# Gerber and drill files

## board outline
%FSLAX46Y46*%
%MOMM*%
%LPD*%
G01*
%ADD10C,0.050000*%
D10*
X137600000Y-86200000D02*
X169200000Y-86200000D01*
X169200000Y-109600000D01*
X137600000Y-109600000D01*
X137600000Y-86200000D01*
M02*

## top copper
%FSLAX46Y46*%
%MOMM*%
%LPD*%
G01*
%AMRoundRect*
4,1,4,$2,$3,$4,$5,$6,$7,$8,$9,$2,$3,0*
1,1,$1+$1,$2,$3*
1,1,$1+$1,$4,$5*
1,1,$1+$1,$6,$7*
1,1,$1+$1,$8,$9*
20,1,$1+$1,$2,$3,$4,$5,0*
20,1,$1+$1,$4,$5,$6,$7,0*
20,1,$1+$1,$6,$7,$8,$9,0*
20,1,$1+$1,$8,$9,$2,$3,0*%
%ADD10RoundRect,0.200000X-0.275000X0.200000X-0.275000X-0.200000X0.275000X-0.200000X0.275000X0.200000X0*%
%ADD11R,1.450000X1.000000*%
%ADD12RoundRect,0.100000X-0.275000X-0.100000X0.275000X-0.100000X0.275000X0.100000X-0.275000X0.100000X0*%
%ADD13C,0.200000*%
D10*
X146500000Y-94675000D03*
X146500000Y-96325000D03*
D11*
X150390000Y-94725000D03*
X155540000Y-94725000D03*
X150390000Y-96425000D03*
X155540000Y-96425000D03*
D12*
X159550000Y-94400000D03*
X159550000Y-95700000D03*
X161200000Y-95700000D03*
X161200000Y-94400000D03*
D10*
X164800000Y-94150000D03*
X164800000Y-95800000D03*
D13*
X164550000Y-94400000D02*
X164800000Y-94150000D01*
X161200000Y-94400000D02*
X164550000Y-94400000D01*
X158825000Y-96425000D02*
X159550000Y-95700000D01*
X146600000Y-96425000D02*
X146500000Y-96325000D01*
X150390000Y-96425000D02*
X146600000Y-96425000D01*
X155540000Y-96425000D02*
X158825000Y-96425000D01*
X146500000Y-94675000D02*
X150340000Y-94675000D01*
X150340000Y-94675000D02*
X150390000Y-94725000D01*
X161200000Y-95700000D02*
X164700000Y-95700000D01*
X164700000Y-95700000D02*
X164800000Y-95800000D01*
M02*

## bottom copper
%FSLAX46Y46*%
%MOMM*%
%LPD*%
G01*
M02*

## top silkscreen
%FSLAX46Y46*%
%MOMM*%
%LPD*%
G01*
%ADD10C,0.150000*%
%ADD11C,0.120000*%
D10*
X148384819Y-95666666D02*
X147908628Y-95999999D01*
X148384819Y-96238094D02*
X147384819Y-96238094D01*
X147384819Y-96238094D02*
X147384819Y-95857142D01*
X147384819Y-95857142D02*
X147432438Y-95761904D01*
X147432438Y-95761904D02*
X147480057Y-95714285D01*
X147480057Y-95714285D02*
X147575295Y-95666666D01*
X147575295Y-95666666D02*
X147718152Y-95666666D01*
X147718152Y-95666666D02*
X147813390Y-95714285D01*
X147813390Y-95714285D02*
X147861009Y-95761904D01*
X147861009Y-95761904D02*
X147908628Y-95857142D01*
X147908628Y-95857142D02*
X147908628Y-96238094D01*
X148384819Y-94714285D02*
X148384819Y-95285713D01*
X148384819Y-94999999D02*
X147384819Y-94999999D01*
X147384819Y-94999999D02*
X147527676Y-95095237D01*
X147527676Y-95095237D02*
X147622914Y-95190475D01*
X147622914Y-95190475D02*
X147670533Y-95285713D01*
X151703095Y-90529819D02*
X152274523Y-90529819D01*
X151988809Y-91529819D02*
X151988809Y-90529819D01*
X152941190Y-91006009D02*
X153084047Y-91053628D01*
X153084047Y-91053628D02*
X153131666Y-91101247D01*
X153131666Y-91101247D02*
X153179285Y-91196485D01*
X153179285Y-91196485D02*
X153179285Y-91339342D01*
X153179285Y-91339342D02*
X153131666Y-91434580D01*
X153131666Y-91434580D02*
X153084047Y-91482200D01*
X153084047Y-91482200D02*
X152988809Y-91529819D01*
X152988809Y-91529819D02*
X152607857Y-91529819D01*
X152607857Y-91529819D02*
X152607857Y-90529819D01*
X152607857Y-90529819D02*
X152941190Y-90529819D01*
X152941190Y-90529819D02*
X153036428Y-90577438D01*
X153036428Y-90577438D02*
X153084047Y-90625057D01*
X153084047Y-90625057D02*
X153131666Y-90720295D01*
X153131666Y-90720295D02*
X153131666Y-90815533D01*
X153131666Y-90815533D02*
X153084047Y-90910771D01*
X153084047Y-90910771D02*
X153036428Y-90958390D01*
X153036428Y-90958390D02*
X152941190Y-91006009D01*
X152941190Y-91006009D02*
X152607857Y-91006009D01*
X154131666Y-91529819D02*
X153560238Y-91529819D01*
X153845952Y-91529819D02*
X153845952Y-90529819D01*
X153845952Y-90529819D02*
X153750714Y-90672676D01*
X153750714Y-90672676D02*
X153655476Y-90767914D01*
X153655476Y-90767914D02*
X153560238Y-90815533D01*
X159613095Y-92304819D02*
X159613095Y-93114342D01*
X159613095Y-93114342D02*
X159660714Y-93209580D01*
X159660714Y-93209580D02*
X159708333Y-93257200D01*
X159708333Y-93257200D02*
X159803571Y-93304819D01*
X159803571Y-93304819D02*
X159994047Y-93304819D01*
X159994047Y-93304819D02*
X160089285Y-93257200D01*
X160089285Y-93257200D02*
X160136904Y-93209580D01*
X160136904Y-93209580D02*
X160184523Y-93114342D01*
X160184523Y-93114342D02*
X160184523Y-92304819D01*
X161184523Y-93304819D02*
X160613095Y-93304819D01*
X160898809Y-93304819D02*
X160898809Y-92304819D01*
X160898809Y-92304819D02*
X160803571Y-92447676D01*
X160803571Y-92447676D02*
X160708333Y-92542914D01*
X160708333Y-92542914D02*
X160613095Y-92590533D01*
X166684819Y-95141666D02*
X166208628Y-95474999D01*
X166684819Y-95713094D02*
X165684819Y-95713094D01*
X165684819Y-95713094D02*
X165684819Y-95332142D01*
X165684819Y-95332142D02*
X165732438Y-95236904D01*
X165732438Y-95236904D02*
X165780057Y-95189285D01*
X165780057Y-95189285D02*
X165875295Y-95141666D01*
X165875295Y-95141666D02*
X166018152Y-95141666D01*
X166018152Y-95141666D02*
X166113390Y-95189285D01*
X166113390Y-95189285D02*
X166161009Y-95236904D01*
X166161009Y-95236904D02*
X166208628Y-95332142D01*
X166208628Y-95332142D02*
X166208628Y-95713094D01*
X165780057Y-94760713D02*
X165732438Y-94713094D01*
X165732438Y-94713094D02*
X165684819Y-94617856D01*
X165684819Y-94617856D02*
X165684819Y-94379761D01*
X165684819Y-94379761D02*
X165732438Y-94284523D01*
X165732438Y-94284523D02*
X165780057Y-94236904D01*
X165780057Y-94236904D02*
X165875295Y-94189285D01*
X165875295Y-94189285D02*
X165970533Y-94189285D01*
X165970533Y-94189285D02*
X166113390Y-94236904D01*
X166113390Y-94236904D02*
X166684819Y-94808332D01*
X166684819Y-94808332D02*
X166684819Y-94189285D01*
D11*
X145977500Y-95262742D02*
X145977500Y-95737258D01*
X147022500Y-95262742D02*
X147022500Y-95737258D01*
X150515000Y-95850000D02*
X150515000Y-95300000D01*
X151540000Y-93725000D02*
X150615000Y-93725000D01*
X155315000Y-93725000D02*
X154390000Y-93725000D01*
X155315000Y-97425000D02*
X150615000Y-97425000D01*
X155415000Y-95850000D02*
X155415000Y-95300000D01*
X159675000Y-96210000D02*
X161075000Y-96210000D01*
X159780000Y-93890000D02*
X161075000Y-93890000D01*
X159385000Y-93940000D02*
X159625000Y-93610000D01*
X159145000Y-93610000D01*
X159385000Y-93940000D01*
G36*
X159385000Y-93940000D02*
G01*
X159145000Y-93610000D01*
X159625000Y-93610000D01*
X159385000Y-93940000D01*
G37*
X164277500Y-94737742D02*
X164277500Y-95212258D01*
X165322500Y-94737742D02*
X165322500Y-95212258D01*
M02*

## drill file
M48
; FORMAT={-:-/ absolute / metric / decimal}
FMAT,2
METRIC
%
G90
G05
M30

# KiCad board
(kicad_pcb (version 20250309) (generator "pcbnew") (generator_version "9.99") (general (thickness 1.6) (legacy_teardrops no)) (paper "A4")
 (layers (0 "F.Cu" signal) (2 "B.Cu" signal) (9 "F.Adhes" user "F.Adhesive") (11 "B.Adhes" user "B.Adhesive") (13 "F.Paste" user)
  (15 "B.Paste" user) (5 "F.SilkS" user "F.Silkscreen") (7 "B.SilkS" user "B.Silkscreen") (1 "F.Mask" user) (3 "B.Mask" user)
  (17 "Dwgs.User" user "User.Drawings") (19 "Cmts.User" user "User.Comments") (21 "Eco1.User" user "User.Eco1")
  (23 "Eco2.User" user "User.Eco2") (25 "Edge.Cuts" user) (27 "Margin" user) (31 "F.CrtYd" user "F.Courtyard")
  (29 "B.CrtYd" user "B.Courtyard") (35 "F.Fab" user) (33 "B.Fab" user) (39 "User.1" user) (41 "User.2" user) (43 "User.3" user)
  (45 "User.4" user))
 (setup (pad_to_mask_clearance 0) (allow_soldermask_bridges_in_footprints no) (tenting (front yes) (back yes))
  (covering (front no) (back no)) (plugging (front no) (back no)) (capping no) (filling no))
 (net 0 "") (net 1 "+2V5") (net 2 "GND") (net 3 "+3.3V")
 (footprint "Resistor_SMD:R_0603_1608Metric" (layer "F.Cu") (at 146.5 95.5 -90)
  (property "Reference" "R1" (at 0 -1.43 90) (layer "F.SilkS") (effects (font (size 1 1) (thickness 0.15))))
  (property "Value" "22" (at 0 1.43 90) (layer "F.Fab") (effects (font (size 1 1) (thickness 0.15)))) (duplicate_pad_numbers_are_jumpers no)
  (fp_line (start -0.237258 0.5225) (end 0.237258 0.5225) (stroke (width 0.12) (type solid)) (layer "F.SilkS"))
  (fp_line (start -0.237258 -0.5225) (end 0.237258 -0.5225) (stroke (width 0.12) (type solid)) (layer "F.SilkS"))
  (pad "1" smd roundrect (at -0.825 0 270) (size 0.8 0.95) (layers "F.Cu" "F.Mask" "F.Paste") (roundrect_rratio 0.25) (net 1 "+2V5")
   (tenting (front none) (back none)))
  (pad "2" smd roundrect (at 0.825 0 270) (size 0.8 0.95) (layers "F.Cu" "F.Mask" "F.Paste") (roundrect_rratio 0.25) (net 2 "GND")
   (tenting (front none) (back none))))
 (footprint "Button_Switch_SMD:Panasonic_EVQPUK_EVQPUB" (layer "F.Cu") (at 152.965 95.575)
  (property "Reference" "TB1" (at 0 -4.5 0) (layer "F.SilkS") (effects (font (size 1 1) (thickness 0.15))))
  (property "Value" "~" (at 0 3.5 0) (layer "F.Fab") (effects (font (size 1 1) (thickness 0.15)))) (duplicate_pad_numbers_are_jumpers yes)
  (fp_line (start -2.45 0.275) (end -2.45 -0.275) (stroke (width 0.12) (type solid)) (layer "F.SilkS"))
  (fp_line (start -1.425 -1.85) (end -2.35 -1.85) (stroke (width 0.12) (type solid)) (layer "F.SilkS"))
  (fp_line (start 2.35 -1.85) (end 1.425 -1.85) (stroke (width 0.12) (type solid)) (layer "F.SilkS"))
  (fp_line (start 2.35 1.85) (end -2.35 1.85) (stroke (width 0.12) (type solid)) (layer "F.SilkS"))
  (fp_line (start 2.45 0.275) (end 2.45 -0.275) (stroke (width 0.12) (type solid)) (layer "F.SilkS"))
  (pad "1" smd rect (at -2.575 -0.85 180) (size 1.45 1) (layers "F.Cu" "F.Mask" "F.Paste") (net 1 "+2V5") (tenting (front none) (back none)))
  (pad "1" smd rect (at 2.575 -0.85 180) (size 1.45 1) (layers "F.Cu" "F.Mask" "F.Paste") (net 1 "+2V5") (tenting (front none) (back none)))
  (pad "2" smd rect (at -2.575 0.85 180) (size 1.45 1) (layers "F.Cu" "F.Mask" "F.Paste") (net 2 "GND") (tenting (front none) (back none)))
  (pad "2" smd rect (at 2.575 0.85 180) (size 1.45 1) (layers "F.Cu" "F.Mask" "F.Paste") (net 2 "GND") (tenting (front none) (back none))))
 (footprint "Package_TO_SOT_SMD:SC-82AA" (layer "F.Cu") (at 160.375 95.05)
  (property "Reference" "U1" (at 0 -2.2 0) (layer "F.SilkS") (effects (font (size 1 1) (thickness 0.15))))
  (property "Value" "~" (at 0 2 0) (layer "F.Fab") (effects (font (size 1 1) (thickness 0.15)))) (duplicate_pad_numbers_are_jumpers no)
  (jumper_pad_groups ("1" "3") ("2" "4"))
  (fp_line (start -0.7 1.16) (end 0.7 1.16) (stroke (width 0.12) (type solid)) (layer "F.SilkS"))
  (fp_line (start -0.595 -1.16) (end 0.7 -1.16) (stroke (width 0.12) (type solid)) (layer "F.SilkS"))
  (fp_poly
   (pts (xy -0.99 -1.11) (xy -0.75 -1.44) (xy -1.23 -1.44) (xy -0.99 -1.11)) (stroke (width 0.12) (type solid)) (fill yes) (layer "F.SilkS"))
  (pad "1" smd roundrect (at -0.825 -0.65) (size 0.75 0.4) (layers "F.Cu" "F.Mask" "F.Paste") (roundrect_rratio 0.25) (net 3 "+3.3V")
   (tenting (front none) (back none)))
  (pad "2" smd roundrect (at -0.825 0.65) (size 0.75 0.4) (layers "F.Cu" "F.Mask" "F.Paste") (roundrect_rratio 0.25) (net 2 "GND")
   (tenting (front none) (back none)))
  (pad "3" smd roundrect (at 0.825 0.65) (size 0.75 0.4) (layers "F.Cu" "F.Mask" "F.Paste") (roundrect_rratio 0.25) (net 3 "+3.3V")
   (tenting (front none) (back none)))
  (pad "4" smd roundrect (at 0.825 -0.65) (size 0.75 0.4) (layers "F.Cu" "F.Mask" "F.Paste") (roundrect_rratio 0.25) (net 2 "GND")
   (tenting (front none) (back none))))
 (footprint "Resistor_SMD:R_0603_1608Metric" (layer "F.Cu") (at 164.8 94.975 -90)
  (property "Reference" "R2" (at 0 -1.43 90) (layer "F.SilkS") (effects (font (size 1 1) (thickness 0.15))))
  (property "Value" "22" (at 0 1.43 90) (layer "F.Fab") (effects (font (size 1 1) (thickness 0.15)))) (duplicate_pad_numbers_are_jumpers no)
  (fp_line (start -0.237258 0.5225) (end 0.237258 0.5225) (stroke (width 0.12) (type solid)) (layer "F.SilkS"))
  (fp_line (start -0.237258 -0.5225) (end 0.237258 -0.5225) (stroke (width 0.12) (type solid)) (layer "F.SilkS"))
  (pad "1" smd roundrect (at -0.825 0 270) (size 0.8 0.95) (layers "F.Cu" "F.Mask" "F.Paste") (roundrect_rratio 0.25) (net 2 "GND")
   (tenting (front none) (back none)))
  (pad "2" smd roundrect (at 0.825 0 270) (size 0.8 0.95) (layers "F.Cu" "F.Mask" "F.Paste") (roundrect_rratio 0.25) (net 3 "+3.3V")
   (tenting (front none) (back none))))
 (gr_rect (start 137.6 86.2) (end 169.2 109.6) (stroke (width 0.05) (type default)) (fill no) (layer "Edge.Cuts"))
 (segment (start 164.55 94.4) (end 164.8 94.15) (width 0.2) (layer "F.Cu") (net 2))
 (segment (start 161.2 94.4) (end 164.55 94.4) (width 0.2) (layer "F.Cu") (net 2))
 (segment (start 158.825 96.425) (end 159.55 95.7) (width 0.2) (layer "F.Cu") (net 2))
 (segment (start 146.6 96.425) (end 146.5 96.325) (width 0.2) (layer "F.Cu") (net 2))
 (segment (start 150.39 96.425) (end 146.6 96.425) (width 0.2) (layer "F.Cu") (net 2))
 (segment (start 155.54 96.425) (end 158.825 96.425) (width 0.2) (layer "F.Cu") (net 2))
 (segment (start 146.5 94.675) (end 150.34 94.675) (width 0.2) (layer "F.Cu") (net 1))
 (segment (start 150.34 94.675) (end 150.39 94.725) (width 0.2) (layer "F.Cu") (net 1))
 (segment (start 161.2 95.7) (end 164.7 95.7) (width 0.2) (layer "F.Cu") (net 3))
 (segment (start 164.7 95.7) (end 164.8 95.8) (width 0.2) (layer "F.Cu") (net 3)))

